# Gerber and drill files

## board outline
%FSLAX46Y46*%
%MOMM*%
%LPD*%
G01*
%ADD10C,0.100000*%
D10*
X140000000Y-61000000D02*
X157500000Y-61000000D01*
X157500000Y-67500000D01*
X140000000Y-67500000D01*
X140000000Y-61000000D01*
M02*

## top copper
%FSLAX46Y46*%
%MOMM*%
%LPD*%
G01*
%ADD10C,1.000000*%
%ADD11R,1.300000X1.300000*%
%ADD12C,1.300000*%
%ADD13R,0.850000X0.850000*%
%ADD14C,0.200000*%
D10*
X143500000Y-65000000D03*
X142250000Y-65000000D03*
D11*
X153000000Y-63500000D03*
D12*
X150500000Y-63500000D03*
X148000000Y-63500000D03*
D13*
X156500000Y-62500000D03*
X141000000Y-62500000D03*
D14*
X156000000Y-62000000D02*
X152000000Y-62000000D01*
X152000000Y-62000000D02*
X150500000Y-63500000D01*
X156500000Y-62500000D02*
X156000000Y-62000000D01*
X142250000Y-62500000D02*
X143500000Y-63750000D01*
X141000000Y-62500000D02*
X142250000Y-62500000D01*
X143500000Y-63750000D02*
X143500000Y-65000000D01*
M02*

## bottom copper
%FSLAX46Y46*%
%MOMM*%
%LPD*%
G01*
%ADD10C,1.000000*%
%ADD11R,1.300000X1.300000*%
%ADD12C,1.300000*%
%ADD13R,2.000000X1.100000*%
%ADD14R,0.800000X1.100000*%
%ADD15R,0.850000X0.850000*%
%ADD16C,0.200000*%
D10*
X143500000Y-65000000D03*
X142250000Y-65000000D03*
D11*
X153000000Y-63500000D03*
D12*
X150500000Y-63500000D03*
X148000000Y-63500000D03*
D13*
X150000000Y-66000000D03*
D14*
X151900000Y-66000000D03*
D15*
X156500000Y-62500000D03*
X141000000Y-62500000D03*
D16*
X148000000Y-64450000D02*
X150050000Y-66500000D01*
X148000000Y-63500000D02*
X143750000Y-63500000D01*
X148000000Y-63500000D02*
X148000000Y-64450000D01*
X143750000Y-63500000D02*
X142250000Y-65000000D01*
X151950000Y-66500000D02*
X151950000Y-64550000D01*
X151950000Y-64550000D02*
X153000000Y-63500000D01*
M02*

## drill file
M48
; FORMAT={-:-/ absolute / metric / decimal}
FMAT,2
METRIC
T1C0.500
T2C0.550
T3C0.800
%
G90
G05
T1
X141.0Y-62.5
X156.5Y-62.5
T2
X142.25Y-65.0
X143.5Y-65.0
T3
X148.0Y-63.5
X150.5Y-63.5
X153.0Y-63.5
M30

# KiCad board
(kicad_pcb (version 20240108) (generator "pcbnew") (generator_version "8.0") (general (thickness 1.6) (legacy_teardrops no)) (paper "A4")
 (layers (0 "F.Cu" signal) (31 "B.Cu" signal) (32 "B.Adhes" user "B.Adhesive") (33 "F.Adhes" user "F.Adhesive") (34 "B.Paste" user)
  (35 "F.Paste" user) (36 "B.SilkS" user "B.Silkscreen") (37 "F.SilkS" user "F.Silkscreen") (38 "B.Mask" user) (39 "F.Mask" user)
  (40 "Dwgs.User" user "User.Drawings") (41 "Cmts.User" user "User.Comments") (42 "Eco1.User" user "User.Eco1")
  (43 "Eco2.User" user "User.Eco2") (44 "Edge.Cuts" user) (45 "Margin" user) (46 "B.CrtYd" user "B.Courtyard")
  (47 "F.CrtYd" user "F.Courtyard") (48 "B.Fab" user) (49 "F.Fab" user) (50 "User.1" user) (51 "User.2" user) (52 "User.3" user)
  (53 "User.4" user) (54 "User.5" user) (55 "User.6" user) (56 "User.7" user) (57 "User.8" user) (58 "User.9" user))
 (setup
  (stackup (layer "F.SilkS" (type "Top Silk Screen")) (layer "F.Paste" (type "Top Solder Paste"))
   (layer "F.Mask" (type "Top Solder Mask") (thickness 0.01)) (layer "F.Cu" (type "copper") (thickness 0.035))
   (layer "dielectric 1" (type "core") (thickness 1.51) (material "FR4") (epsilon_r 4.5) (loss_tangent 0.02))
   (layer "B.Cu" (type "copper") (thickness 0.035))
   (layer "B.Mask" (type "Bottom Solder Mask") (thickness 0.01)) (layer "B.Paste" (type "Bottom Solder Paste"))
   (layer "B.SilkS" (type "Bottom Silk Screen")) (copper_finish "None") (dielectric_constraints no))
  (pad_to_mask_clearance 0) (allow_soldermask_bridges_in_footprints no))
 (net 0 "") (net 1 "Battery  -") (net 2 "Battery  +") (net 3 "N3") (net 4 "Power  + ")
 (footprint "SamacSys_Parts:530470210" (layer "F.Cu") (at 143.5 65)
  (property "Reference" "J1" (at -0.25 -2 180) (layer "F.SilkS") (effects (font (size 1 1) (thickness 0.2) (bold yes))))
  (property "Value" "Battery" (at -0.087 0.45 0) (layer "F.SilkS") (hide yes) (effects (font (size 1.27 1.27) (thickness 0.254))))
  (pad "1" thru_hole circle (at 0 0) (size 1 1) (drill 0.55) (layers "*.Cu" "*.Mask") (remove_unused_layers no) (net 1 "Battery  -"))
  (pad "2" thru_hole circle (at -1.25 0) (size 1 1) (drill 0.55) (layers "*.Cu" "*.Mask") (remove_unused_layers no) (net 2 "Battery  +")))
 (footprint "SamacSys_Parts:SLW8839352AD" (layer "F.Cu") (at 153 63.5 180)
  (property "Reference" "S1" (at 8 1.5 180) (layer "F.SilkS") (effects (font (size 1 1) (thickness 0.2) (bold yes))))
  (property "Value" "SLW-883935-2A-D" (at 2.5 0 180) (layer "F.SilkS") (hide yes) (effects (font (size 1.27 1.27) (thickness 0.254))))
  (pad "1" thru_hole rect (at 0 0 180) (size 1.3 1.3) (drill 0.8) (layers "*.Cu" "*.Mask") (remove_unused_layers no) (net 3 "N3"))
  (pad "2" thru_hole circle (at 2.5 0 180) (size 1.3 1.3) (drill 0.8) (layers "*.Cu" "*.Mask") (remove_unused_layers no) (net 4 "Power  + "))
  (pad "3" thru_hole circle (at 5 0 180) (size 1.3 1.3) (drill 0.8) (layers "*.Cu" "*.Mask") (remove_unused_layers no) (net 2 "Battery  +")))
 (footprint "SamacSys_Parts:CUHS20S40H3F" (layer "B.Cu") (at 150.95 66)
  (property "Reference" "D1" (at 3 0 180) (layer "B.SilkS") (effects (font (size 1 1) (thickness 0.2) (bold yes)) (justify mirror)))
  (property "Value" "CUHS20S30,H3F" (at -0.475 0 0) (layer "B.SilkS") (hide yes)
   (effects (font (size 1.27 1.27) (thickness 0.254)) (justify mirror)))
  (pad "1" smd rect (at -0.95 0 270) (size 1.1 2) (layers "B.Cu" "B.Paste" "B.Mask") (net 2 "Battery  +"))
  (pad "2" smd rect (at 0.95 0) (size 0.8 1.1) (layers "B.Cu" "B.Paste" "B.Mask") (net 3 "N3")))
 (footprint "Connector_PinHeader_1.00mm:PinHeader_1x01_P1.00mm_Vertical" (layer "B.Cu") (at 156.5 62.5 180)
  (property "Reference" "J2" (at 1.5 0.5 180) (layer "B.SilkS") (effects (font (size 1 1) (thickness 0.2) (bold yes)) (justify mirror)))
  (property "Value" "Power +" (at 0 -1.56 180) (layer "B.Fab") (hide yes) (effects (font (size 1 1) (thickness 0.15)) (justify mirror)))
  (pad "1" thru_hole rect (at 0 0 180) (size 0.85 0.85) (drill 0.5) (layers "*.Cu" "*.Mask") (remove_unused_layers no) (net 4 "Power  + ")))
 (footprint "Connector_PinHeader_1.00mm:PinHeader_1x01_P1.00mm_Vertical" (layer "B.Cu") (at 141 62.5 180)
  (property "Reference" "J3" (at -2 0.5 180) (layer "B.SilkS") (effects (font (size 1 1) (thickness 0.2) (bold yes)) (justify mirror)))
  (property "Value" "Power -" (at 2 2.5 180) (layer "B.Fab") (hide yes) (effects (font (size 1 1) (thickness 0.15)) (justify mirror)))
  (pad "1" thru_hole rect (at 0 0 180) (size 0.85 0.85) (drill 0.5) (layers "*.Cu" "*.Mask") (remove_unused_layers no) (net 1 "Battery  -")))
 (gr_rect (start 140 61) (end 157.5 67.5) (stroke (width 0.1) (type default)) (fill none) (layer "Edge.Cuts"))
 (segment (start 148 64.45) (end 150.05 66.5) (width 0.2) (layer "B.Cu") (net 2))
 (segment (start 148 63.5) (end 143.75 63.5) (width 0.2) (layer "B.Cu") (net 2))
 (segment (start 148 63.5) (end 148 64.45) (width 0.2) (layer "B.Cu") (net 2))
 (segment (start 143.75 63.5) (end 142.25 65) (width 0.2) (layer "B.Cu") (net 2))
 (segment (start 156 62) (end 152 62) (width 0.2) (layer "F.Cu") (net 4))
 (segment (start 152 62) (end 150.5 63.5) (width 0.2) (layer "F.Cu") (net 4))
 (segment (start 156.5 62.5) (end 156 62) (width 0.2) (layer "F.Cu") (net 4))
 (segment (start 142.25 62.5) (end 143.5 63.75) (width 0.2) (layer "F.Cu") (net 1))
 (segment (start 141 62.5) (end 142.25 62.5) (width 0.2) (layer "F.Cu") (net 1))
 (segment (start 143.5 63.75) (end 143.5 65) (width 0.2) (layer "F.Cu") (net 1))
 (segment (start 151.95 66.5) (end 151.95 64.55) (width 0.2) (layer "B.Cu") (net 3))
 (segment (start 151.95 64.55) (end 153 63.5) (width 0.2) (layer "B.Cu") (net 3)))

